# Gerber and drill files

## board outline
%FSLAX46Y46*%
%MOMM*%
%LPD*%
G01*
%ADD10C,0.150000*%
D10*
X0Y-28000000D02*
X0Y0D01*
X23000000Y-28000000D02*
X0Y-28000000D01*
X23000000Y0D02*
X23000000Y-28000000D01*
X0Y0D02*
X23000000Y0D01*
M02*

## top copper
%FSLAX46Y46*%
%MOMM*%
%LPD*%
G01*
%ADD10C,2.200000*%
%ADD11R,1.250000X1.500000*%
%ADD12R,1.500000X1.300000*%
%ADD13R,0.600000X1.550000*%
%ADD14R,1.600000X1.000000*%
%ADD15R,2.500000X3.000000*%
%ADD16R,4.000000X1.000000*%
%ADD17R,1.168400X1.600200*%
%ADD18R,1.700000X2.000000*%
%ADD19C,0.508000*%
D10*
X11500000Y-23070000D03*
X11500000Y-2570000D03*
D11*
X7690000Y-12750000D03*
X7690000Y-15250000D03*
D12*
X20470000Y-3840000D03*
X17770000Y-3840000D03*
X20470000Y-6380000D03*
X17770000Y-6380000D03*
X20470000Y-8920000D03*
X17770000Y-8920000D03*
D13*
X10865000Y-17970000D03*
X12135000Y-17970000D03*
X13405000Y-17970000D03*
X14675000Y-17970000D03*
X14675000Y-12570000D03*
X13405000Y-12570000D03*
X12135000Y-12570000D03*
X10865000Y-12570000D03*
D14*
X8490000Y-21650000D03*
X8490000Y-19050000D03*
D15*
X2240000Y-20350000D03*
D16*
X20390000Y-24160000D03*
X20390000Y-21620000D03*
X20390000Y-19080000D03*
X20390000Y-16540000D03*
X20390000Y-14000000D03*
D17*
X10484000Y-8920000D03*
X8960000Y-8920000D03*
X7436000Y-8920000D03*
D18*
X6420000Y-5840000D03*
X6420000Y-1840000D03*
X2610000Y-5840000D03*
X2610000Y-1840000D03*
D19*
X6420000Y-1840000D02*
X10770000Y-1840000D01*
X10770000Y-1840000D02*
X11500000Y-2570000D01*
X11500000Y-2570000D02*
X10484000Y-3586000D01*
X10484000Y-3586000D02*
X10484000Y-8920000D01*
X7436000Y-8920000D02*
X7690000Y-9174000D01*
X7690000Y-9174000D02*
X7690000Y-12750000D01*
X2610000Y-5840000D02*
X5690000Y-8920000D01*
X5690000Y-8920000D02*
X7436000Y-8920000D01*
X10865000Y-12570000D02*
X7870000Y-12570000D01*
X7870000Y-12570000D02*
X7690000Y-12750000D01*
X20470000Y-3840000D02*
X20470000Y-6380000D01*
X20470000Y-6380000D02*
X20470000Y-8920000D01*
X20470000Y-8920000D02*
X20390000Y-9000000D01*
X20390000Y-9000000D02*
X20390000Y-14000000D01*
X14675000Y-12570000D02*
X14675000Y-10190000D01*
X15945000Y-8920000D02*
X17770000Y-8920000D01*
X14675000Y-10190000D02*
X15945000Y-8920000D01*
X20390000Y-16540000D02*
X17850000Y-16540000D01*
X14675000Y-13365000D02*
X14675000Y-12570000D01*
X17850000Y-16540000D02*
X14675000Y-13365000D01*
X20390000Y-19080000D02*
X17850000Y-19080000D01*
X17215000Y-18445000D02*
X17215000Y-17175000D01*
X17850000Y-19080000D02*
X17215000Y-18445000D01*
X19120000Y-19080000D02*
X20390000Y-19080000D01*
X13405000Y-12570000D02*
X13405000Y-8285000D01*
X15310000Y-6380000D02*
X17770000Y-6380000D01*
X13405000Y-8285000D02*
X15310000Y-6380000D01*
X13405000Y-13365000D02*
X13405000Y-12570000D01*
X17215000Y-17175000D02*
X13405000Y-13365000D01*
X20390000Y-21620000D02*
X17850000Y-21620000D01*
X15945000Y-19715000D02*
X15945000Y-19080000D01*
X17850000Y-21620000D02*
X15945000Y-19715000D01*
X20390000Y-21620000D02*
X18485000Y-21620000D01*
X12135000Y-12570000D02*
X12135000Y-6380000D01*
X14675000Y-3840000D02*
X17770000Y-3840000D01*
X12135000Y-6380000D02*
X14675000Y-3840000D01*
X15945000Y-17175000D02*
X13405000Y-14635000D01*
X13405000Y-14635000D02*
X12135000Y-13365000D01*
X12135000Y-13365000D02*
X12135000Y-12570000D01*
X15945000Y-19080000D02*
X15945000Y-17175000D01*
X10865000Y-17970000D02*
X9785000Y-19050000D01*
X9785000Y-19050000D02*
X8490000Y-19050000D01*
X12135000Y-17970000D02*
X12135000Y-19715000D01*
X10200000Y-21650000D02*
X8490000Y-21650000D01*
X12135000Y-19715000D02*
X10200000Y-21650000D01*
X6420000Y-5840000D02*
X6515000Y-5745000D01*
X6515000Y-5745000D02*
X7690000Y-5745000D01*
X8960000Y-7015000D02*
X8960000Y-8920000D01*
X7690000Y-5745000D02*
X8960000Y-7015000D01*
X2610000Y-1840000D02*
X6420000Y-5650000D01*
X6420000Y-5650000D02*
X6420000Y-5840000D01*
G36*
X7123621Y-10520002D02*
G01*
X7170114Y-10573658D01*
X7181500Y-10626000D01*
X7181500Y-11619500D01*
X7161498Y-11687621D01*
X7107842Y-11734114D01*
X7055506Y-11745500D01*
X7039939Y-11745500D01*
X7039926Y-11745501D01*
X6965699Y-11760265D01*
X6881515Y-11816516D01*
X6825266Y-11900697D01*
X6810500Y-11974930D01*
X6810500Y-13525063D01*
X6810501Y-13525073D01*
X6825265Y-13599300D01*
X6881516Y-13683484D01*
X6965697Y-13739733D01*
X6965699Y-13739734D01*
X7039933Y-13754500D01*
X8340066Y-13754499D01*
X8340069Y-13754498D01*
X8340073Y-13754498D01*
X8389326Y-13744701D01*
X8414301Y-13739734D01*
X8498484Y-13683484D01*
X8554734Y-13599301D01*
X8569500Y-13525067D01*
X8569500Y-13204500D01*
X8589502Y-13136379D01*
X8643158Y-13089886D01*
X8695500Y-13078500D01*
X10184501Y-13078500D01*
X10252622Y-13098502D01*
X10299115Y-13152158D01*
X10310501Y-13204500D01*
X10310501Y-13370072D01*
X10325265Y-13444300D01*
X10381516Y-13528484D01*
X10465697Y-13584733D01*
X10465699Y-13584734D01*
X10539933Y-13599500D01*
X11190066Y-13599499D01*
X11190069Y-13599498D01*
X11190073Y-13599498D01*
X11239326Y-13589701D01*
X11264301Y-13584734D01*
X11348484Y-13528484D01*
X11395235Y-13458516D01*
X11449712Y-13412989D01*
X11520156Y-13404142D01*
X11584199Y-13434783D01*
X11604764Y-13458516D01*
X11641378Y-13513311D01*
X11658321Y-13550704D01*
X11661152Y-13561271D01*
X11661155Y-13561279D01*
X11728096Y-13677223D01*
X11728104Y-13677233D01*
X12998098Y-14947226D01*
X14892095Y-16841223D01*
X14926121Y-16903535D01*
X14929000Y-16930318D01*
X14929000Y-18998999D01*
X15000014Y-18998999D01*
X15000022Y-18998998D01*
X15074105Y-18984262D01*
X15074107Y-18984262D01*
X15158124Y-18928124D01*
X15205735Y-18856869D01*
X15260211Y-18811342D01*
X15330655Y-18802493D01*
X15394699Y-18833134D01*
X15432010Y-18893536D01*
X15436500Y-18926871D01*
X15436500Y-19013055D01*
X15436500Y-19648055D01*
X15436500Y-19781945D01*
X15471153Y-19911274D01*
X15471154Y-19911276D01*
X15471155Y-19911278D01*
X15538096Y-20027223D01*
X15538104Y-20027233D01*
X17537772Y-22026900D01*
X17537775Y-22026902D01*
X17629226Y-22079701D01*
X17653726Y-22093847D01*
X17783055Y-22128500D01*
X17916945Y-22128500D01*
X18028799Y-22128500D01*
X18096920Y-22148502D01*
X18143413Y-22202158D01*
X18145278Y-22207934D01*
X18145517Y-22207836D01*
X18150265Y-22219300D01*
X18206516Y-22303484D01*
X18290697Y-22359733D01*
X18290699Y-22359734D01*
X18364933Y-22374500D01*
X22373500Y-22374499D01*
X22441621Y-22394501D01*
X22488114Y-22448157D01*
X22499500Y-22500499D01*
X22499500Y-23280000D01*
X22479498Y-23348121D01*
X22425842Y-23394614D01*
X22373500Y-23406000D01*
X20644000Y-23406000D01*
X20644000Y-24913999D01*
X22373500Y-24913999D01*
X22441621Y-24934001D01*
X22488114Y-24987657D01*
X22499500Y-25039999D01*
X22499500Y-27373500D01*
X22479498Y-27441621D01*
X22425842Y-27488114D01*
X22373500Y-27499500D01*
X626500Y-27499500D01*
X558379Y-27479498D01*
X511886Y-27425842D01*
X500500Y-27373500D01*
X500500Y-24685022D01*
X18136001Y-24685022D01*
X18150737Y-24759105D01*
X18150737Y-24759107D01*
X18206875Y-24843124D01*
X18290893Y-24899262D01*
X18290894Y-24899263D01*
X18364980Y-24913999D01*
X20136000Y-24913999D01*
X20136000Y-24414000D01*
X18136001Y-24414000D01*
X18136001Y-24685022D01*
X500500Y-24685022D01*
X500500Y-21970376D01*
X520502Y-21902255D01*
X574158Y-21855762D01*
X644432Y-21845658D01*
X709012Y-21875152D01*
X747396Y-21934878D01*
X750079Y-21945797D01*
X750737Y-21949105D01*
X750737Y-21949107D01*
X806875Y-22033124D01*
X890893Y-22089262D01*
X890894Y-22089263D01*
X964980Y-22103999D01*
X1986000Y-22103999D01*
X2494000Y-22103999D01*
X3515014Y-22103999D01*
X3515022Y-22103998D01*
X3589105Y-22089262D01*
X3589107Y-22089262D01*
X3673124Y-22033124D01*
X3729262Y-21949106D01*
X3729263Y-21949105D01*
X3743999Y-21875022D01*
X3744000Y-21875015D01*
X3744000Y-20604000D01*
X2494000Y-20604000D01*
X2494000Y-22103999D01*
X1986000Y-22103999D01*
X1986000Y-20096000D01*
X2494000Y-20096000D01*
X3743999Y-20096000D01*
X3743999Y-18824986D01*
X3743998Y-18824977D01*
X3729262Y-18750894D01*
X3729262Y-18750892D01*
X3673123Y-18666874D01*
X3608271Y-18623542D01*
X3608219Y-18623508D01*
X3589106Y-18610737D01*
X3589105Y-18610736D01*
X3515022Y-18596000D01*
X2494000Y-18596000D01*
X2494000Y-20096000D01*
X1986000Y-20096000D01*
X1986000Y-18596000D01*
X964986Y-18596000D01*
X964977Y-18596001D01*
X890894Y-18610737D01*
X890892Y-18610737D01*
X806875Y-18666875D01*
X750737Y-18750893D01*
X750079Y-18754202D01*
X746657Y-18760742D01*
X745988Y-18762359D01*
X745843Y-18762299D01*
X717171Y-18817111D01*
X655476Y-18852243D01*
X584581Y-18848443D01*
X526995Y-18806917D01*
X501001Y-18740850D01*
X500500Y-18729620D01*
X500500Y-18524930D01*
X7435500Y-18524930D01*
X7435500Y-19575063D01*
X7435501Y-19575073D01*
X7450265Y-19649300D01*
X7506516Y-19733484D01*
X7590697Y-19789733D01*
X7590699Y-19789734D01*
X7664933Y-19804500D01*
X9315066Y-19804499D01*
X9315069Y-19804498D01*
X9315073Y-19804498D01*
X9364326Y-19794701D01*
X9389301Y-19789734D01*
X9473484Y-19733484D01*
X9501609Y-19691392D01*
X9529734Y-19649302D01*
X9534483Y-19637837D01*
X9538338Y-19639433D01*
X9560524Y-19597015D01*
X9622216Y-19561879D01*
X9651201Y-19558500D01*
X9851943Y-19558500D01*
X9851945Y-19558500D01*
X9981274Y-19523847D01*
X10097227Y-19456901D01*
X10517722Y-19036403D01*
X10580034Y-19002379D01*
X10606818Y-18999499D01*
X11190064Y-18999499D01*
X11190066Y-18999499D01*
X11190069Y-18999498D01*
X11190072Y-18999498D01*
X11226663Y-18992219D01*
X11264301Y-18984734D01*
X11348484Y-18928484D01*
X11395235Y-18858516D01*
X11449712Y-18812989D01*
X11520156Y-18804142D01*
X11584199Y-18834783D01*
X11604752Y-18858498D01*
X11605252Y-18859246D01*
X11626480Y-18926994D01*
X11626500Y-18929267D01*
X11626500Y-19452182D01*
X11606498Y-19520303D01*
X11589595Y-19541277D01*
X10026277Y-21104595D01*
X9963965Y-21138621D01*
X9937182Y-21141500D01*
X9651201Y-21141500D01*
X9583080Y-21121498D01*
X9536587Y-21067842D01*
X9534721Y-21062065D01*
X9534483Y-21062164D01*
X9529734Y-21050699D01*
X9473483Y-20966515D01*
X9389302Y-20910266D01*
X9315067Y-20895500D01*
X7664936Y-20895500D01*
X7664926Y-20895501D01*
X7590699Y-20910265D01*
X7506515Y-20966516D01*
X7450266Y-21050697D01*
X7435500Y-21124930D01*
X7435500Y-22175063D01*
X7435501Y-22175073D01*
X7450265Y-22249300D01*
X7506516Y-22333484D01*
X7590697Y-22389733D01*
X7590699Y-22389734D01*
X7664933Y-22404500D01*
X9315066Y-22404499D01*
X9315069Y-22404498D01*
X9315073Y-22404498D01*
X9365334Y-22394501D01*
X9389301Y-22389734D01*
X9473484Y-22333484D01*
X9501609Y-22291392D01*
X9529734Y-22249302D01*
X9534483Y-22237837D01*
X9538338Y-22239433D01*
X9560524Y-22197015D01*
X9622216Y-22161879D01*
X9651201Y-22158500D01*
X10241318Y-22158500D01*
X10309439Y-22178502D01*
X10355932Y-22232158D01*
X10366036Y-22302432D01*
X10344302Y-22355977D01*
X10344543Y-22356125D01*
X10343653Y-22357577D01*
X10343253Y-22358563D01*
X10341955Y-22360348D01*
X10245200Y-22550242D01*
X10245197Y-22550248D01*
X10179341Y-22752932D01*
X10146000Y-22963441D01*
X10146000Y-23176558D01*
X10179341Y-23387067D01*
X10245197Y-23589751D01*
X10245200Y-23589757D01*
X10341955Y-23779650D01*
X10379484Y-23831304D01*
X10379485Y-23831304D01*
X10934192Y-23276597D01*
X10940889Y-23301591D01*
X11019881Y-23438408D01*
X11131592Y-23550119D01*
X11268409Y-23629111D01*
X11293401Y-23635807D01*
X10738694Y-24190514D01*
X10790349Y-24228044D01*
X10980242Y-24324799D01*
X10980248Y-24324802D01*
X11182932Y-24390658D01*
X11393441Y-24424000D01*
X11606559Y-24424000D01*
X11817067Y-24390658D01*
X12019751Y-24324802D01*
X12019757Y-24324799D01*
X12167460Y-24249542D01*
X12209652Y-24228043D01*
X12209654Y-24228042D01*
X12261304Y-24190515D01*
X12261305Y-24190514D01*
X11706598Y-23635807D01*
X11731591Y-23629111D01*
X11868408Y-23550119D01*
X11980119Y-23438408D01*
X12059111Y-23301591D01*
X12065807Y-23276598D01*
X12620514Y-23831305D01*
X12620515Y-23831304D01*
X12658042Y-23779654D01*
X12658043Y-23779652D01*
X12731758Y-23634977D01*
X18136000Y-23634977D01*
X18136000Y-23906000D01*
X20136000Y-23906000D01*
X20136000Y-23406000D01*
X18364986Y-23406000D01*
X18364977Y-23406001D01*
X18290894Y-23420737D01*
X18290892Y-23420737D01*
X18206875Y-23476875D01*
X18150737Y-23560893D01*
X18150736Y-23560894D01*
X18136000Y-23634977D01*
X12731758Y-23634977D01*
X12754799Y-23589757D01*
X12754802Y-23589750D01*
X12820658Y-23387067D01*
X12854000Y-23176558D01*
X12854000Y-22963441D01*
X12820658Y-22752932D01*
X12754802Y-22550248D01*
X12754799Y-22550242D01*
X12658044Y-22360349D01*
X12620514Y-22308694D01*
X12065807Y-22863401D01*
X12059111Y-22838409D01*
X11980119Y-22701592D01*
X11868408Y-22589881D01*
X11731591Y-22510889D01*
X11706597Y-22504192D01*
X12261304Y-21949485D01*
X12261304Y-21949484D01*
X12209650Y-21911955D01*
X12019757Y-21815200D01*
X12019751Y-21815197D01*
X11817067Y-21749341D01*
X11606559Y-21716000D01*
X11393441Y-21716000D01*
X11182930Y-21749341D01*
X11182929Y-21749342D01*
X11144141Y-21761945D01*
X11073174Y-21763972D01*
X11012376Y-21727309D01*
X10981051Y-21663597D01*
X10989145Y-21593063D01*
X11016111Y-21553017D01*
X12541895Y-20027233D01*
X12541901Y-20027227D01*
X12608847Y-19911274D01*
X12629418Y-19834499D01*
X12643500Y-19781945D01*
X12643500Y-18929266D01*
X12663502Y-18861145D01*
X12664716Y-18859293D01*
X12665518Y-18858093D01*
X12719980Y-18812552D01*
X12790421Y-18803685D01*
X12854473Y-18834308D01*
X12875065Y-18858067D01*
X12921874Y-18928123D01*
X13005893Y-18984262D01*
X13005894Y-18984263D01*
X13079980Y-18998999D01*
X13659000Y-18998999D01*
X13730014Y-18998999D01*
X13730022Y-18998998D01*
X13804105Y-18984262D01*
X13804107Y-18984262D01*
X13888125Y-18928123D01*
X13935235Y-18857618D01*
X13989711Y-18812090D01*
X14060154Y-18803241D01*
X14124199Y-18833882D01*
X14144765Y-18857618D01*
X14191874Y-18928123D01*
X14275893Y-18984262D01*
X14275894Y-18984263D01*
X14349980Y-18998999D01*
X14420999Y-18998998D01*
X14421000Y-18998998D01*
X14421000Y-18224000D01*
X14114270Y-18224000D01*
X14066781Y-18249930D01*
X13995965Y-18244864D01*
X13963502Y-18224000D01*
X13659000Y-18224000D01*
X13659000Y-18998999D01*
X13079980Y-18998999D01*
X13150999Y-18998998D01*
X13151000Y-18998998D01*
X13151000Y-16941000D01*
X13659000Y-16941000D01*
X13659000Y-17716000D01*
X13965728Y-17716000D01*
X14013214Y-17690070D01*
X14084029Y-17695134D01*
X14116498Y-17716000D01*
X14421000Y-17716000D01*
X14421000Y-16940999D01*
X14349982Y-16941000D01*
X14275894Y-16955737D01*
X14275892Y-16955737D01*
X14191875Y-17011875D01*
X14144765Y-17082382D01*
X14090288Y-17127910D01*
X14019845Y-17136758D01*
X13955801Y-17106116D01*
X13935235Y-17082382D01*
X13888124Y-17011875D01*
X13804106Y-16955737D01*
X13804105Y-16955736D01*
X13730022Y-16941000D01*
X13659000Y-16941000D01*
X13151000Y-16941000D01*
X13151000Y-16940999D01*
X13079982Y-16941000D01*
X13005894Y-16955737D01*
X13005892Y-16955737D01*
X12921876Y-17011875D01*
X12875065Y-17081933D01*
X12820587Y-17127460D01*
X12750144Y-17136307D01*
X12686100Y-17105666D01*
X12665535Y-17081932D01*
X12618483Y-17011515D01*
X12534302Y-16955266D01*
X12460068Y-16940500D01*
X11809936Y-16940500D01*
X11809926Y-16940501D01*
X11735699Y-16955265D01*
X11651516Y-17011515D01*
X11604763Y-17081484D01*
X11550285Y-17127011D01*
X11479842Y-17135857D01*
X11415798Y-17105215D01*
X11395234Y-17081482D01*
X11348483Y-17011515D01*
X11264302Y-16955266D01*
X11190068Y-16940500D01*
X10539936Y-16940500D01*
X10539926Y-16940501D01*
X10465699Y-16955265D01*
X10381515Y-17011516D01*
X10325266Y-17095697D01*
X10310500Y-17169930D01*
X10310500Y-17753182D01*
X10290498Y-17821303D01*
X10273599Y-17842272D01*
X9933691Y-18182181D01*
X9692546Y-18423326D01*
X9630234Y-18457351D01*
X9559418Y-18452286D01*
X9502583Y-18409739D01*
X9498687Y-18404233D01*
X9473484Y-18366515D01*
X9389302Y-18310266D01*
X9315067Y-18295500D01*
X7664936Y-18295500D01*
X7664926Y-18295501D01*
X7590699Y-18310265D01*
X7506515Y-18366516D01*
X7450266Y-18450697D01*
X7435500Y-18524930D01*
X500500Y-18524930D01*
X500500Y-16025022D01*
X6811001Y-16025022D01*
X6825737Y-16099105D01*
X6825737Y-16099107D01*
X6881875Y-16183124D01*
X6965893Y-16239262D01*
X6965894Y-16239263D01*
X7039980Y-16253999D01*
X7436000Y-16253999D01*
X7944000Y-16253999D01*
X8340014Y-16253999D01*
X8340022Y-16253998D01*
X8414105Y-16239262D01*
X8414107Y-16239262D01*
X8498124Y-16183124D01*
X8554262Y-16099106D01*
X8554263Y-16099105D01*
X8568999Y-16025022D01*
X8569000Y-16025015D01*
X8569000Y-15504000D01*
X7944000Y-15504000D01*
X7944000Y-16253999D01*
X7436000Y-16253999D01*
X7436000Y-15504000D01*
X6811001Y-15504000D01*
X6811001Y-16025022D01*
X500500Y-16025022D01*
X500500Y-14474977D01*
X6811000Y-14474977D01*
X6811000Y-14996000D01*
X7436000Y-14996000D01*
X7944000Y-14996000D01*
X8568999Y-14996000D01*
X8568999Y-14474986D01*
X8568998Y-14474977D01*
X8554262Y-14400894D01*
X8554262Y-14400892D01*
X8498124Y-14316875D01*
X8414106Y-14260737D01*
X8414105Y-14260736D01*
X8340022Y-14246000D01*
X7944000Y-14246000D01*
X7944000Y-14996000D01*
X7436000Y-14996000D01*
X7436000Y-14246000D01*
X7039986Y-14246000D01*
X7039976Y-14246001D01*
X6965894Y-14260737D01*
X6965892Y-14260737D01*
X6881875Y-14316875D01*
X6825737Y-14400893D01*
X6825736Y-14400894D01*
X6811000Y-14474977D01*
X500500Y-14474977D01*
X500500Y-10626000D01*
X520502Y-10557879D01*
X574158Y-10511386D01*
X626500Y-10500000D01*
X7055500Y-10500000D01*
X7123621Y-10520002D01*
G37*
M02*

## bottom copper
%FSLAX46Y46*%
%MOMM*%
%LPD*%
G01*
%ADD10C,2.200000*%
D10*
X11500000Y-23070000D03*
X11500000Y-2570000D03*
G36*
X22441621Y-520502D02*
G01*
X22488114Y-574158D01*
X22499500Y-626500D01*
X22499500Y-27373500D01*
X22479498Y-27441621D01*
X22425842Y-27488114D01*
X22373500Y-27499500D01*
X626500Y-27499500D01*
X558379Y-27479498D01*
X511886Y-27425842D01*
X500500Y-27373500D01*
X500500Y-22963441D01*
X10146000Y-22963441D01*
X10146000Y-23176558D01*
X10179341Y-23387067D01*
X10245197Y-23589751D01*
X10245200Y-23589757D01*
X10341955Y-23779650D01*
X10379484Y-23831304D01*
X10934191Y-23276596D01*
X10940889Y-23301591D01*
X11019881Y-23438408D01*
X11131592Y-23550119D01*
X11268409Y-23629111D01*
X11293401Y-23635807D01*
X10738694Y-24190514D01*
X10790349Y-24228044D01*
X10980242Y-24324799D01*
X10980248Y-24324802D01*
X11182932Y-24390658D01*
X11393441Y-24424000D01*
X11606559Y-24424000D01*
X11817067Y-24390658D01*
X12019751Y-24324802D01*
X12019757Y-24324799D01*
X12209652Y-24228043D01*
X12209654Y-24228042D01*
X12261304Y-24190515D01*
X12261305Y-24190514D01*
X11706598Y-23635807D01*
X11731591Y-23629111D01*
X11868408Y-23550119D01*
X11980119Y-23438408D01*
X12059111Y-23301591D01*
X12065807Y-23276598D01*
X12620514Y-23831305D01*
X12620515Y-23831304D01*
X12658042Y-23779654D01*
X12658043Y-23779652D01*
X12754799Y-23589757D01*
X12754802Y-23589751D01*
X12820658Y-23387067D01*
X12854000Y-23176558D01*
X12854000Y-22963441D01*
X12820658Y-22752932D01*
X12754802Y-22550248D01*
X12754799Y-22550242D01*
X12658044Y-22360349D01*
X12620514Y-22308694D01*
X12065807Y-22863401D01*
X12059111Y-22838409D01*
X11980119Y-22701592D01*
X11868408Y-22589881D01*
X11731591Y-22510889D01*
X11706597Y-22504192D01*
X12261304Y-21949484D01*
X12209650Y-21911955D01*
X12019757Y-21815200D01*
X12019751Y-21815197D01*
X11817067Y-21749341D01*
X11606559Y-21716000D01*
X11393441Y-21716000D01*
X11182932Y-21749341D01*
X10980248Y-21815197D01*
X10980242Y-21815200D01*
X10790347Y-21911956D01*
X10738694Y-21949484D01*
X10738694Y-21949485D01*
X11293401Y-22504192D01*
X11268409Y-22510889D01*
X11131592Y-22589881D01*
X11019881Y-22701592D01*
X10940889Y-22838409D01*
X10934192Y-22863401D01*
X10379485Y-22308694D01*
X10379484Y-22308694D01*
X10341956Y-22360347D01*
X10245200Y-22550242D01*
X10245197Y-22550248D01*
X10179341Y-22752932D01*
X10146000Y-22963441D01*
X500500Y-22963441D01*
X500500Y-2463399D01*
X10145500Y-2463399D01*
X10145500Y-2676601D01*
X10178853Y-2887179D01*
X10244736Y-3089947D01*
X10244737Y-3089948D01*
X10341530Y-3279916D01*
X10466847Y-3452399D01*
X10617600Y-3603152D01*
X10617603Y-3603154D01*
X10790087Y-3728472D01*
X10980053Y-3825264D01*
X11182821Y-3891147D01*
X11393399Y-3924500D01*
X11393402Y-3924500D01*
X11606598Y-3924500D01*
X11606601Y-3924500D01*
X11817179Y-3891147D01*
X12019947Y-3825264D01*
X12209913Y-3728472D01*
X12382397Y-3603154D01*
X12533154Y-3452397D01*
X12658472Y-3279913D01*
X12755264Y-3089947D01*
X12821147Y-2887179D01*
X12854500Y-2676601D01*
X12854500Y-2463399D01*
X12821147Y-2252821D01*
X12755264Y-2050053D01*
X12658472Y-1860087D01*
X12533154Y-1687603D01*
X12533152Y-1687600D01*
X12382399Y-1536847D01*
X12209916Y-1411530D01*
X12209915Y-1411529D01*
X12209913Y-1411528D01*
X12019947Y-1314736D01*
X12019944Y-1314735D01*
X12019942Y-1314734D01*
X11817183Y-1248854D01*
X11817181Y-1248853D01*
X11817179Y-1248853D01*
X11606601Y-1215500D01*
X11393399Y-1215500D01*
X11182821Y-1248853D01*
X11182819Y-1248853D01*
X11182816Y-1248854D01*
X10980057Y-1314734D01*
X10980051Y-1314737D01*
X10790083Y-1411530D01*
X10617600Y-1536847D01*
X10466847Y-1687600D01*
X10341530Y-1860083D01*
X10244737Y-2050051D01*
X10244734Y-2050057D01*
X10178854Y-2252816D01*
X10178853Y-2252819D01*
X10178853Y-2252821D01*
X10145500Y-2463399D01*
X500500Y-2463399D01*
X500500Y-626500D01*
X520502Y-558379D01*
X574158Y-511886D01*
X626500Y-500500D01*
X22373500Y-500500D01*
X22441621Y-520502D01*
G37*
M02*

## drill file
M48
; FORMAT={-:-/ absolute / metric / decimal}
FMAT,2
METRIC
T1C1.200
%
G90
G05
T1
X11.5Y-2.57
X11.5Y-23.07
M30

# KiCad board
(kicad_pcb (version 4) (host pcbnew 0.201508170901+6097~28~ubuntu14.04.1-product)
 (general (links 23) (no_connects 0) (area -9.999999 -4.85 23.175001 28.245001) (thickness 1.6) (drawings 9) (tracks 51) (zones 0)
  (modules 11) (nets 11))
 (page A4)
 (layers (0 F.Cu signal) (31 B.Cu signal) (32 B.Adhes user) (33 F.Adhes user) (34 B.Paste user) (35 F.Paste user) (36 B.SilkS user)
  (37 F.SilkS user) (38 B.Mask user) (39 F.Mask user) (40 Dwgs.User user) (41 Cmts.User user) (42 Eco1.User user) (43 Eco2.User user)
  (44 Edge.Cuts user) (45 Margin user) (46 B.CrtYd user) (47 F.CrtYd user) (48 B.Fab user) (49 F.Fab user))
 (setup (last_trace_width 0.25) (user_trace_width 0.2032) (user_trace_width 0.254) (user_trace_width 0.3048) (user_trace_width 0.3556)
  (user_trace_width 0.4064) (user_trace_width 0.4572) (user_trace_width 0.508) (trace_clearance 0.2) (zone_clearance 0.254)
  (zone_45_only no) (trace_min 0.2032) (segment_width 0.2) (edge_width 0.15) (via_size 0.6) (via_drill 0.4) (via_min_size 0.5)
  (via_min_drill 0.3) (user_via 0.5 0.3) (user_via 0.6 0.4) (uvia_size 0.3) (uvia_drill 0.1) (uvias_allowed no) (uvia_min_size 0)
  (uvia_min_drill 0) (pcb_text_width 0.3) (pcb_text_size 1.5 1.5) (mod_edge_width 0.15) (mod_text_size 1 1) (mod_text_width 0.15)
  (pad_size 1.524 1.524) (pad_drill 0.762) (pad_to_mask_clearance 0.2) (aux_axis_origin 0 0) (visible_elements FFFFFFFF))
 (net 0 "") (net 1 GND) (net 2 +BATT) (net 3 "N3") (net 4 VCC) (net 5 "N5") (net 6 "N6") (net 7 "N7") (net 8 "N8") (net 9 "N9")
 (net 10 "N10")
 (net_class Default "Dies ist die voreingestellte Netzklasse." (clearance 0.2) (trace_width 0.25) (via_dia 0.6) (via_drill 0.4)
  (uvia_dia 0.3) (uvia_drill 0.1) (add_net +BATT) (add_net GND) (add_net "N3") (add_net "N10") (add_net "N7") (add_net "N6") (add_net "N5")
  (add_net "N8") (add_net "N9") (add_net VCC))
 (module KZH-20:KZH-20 (layer B.Cu) (at 11.5 2.57 90)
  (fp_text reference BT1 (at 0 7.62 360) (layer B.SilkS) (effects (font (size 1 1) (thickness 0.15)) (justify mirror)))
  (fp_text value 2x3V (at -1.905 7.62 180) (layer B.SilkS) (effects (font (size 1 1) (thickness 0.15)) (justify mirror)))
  (pad 2 thru_hole circle (at -20.5 0 90) (size 2.2 2.2) (drill 1.2) (layers *.Cu *.Mask B.SilkS) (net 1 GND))
  (pad 1 thru_hole circle (at 0 0 90) (size 2.2 2.2) (drill 1.2) (layers *.Cu *.Mask B.SilkS) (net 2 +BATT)))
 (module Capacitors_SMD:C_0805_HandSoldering (layer F.Cu) (at 7.69 14 270)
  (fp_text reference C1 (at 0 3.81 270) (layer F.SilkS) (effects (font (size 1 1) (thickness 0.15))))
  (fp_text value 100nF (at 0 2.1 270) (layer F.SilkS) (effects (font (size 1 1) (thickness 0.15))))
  (pad 1 smd rect (at -1.25 0 270) (size 1.5 1.25) (layers F.Cu F.Paste F.Mask) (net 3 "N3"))
  (pad 2 smd rect (at 1.25 0 270) (size 1.5 1.25) (layers F.Cu F.Paste F.Mask) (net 1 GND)))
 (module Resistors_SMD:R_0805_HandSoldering (layer F.Cu) (at 19.12 3.84 180)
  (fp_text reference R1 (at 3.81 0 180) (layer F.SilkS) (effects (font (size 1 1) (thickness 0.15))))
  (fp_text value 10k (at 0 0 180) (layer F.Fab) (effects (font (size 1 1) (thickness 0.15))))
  (pad 1 smd rect (at -1.35 0 180) (size 1.5 1.3) (layers F.Cu F.Paste F.Mask) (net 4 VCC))
  (pad 2 smd rect (at 1.35 0 180) (size 1.5 1.3) (layers F.Cu F.Paste F.Mask) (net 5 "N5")))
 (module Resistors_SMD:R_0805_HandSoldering (layer F.Cu) (at 19.12 6.38 180)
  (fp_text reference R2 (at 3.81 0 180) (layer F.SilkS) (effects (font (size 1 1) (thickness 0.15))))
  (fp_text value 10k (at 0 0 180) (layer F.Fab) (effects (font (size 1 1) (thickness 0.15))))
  (pad 1 smd rect (at -1.35 0 180) (size 1.5 1.3) (layers F.Cu F.Paste F.Mask) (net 4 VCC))
  (pad 2 smd rect (at 1.35 0 180) (size 1.5 1.3) (layers F.Cu F.Paste F.Mask) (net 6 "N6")))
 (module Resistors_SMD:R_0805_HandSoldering (layer F.Cu) (at 19.12 8.92 180)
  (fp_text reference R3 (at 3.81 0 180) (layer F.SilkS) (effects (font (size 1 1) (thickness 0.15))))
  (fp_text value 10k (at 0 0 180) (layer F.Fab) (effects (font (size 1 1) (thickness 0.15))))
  (pad 1 smd rect (at -1.35 0 180) (size 1.5 1.3) (layers F.Cu F.Paste F.Mask) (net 4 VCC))
  (pad 2 smd rect (at 1.35 0 180) (size 1.5 1.3) (layers F.Cu F.Paste F.Mask) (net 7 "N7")))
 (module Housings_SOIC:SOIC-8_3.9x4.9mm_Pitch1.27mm (layer F.Cu) (at 12.77 15.27 90)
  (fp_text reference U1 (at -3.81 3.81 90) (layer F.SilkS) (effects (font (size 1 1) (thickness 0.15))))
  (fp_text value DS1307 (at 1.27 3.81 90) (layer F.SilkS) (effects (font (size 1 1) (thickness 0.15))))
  (pad 1 smd rect (at -2.7 -1.905 90) (size 1.55 0.6) (layers F.Cu F.Paste F.Mask) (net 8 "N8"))
  (pad 2 smd rect (at -2.7 -0.635 90) (size 1.55 0.6) (layers F.Cu F.Paste F.Mask) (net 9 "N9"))
  (pad 3 smd rect (at -2.7 0.635 90) (size 1.55 0.6) (layers F.Cu F.Paste F.Mask) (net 1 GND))
  (pad 4 smd rect (at -2.7 1.905 90) (size 1.55 0.6) (layers F.Cu F.Paste F.Mask) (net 1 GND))
  (pad 5 smd rect (at 2.7 1.905 90) (size 1.55 0.6) (layers F.Cu F.Paste F.Mask) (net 7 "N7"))
  (pad 6 smd rect (at 2.7 0.635 90) (size 1.55 0.6) (layers F.Cu F.Paste F.Mask) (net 6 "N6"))
  (pad 7 smd rect (at 2.7 -0.635 90) (size 1.55 0.6) (layers F.Cu F.Paste F.Mask) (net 5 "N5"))
  (pad 8 smd rect (at 2.7 -1.905 90) (size 1.55 0.6) (layers F.Cu F.Paste F.Mask) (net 3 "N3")))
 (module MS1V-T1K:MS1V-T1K (layer F.Cu) (at 7.69 20.35)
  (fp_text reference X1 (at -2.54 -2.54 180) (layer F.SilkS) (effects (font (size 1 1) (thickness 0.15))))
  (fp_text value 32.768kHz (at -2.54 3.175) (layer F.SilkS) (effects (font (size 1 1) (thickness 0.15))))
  (pad 1 smd rect (at 0.8 1.3) (size 1.6 1) (layers F.Cu F.Paste F.Mask) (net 9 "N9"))
  (pad 2 smd rect (at 0.8 -1.3) (size 1.6 1) (layers F.Cu F.Paste F.Mask) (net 8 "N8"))
  (pad 3 smd rect (at -5.45 0) (size 2.5 3) (layers F.Cu F.Paste F.Mask) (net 1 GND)))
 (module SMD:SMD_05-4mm (layer F.Cu) (at 20.39 14)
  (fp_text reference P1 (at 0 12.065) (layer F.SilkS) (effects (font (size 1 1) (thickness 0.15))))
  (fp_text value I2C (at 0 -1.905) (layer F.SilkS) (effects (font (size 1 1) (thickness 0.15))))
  (pad 5 connect rect (at 0 10.16) (size 4 1) (layers F.Cu F.Mask) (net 1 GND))
  (pad 4 connect rect (at 0 7.62) (size 4 1) (layers F.Cu F.Mask) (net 5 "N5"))
  (pad 3 connect rect (at 0 5.08) (size 4 1) (layers F.Cu F.Mask) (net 6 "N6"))
  (pad 2 connect rect (at 0 2.54) (size 4 1) (layers F.Cu F.Mask) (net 7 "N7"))
  (pad 1 connect rect (at 0 0) (size 4 1) (layers F.Cu F.Mask) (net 4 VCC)))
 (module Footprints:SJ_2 (layer F.Cu) (at 8.96 8.92 180)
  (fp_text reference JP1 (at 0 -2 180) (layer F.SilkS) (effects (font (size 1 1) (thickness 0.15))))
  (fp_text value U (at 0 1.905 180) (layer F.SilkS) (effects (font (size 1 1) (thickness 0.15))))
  (pad 1 smd rect (at -1.524 0 180) (size 1.1684 1.6002) (layers F.Cu F.Paste F.Mask) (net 2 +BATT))
  (pad 2 smd rect (at 0 0 180) (size 1.1684 1.6002) (layers F.Cu F.Paste F.Mask) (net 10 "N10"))
  (pad 3 smd rect (at 1.524 0 180) (size 1.1684 1.6002) (layers F.Cu F.Paste F.Mask) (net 3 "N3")))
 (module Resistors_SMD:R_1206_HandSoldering (layer F.Cu) (at 6.42 3.84 90)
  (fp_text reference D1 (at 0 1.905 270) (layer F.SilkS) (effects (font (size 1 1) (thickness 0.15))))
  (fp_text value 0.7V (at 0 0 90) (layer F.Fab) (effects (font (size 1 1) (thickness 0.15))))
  (pad 1 smd rect (at -2 0 90) (size 2 1.7) (layers F.Cu F.Paste F.Mask) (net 10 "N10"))
  (pad 2 smd rect (at 2 0 90) (size 2 1.7) (layers F.Cu F.Paste F.Mask) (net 2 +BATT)))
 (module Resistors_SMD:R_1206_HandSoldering (layer F.Cu) (at 2.61 3.84 90)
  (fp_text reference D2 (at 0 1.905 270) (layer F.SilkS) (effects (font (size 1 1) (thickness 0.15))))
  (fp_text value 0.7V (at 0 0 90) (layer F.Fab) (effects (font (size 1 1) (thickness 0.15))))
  (pad 1 smd rect (at -2 0 90) (size 2 1.7) (layers F.Cu F.Paste F.Mask) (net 3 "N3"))
  (pad 2 smd rect (at 2 0 90) (size 2 1.7) (layers F.Cu F.Paste F.Mask) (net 10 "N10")))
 (gr_line (start 0 28) (end 0 0) (angle 90) (layer Edge.Cuts) (width 0.15))
 (gr_line (start 23 28) (end 0 28) (angle 90) (layer Edge.Cuts) (width 0.15))
 (gr_line (start 23 0) (end 23 28) (angle 90) (layer Edge.Cuts) (width 0.15))
 (gr_line (start 0 0) (end 23 0) (angle 90) (layer Edge.Cuts) (width 0.15))
 (segment (start 6.42 1.84) (end 10.77 1.84) (width 0.508) (layer F.Cu) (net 2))
 (segment (start 10.77 1.84) (end 11.5 2.57) (width 0.508) (layer F.Cu) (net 2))
 (segment (start 11.5 2.57) (end 10.484 3.586) (width 0.508) (layer F.Cu) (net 2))
 (segment (start 10.484 3.586) (end 10.484 8.92) (width 0.508) (layer F.Cu) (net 2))
 (segment (start 7.436 8.92) (end 7.69 9.174) (width 0.508) (layer F.Cu) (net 3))
 (segment (start 7.69 9.174) (end 7.69 12.75) (width 0.508) (layer F.Cu) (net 3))
 (segment (start 2.61 5.84) (end 5.69 8.92) (width 0.508) (layer F.Cu) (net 3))
 (segment (start 5.69 8.92) (end 7.436 8.92) (width 0.508) (layer F.Cu) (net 3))
 (segment (start 10.865 12.57) (end 7.87 12.57) (width 0.508) (layer F.Cu) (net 3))
 (segment (start 7.87 12.57) (end 7.69 12.75) (width 0.508) (layer F.Cu) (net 3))
 (segment (start 20.47 3.84) (end 20.47 6.38) (width 0.508) (layer F.Cu) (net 4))
 (segment (start 20.47 6.38) (end 20.47 8.92) (width 0.508) (layer F.Cu) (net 4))
 (segment (start 20.47 8.92) (end 20.39 9) (width 0.508) (layer F.Cu) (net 4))
 (segment (start 20.39 9) (end 20.39 14) (width 0.508) (layer F.Cu) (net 4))
 (segment (start 14.675 12.57) (end 14.675 10.19) (width 0.508) (layer F.Cu) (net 7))
 (segment (start 15.945 8.92) (end 17.77 8.92) (width 0.508) (layer F.Cu) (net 7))
 (segment (start 14.675 10.19) (end 15.945 8.92) (width 0.508) (layer F.Cu) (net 7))
 (segment (start 20.39 16.54) (end 17.85 16.54) (width 0.508) (layer F.Cu) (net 7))
 (segment (start 14.675 13.365) (end 14.675 12.57) (width 0.508) (layer F.Cu) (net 7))
 (segment (start 17.85 16.54) (end 14.675 13.365) (width 0.508) (layer F.Cu) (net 7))
 (segment (start 20.39 19.08) (end 17.85 19.08) (width 0.508) (layer F.Cu) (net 6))
 (segment (start 17.215 18.445) (end 17.215 17.175) (width 0.508) (layer F.Cu) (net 6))
 (segment (start 17.85 19.08) (end 17.215 18.445) (width 0.508) (layer F.Cu) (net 6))
 (segment (start 19.12 19.08) (end 20.39 19.08) (width 0.508) (layer F.Cu) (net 6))
 (segment (start 13.405 12.57) (end 13.405 8.285) (width 0.508) (layer F.Cu) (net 6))
 (segment (start 15.31 6.38) (end 17.77 6.38) (width 0.508) (layer F.Cu) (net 6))
 (segment (start 13.405 8.285) (end 15.31 6.38) (width 0.508) (layer F.Cu) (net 6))
 (segment (start 13.405 13.365) (end 13.405 12.57) (width 0.508) (layer F.Cu) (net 6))
 (segment (start 17.215 17.175) (end 13.405 13.365) (width 0.508) (layer F.Cu) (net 6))
 (segment (start 20.39 21.62) (end 17.85 21.62) (width 0.508) (layer F.Cu) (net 5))
 (segment (start 15.945 19.715) (end 15.945 19.08) (width 0.508) (layer F.Cu) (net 5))
 (segment (start 17.85 21.62) (end 15.945 19.715) (width 0.508) (layer F.Cu) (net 5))
 (segment (start 20.39 21.62) (end 18.485 21.62) (width 0.508) (layer F.Cu) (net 5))
 (segment (start 12.135 12.57) (end 12.135 6.38) (width 0.508) (layer F.Cu) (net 5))
 (segment (start 14.675 3.84) (end 17.77 3.84) (width 0.508) (layer F.Cu) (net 5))
 (segment (start 12.135 6.38) (end 14.675 3.84) (width 0.508) (layer F.Cu) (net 5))
 (segment (start 15.945 17.175) (end 13.405 14.635) (width 0.508) (layer F.Cu) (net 5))
 (segment (start 13.405 14.635) (end 12.135 13.365) (width 0.508) (layer F.Cu) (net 5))
 (segment (start 12.135 13.365) (end 12.135 12.57) (width 0.508) (layer F.Cu) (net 5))
 (segment (start 15.945 19.08) (end 15.945 17.175) (width 0.508) (layer F.Cu) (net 5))
 (segment (start 10.865 17.97) (end 9.785 19.05) (width 0.508) (layer F.Cu) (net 8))
 (segment (start 9.785 19.05) (end 8.49 19.05) (width 0.508) (layer F.Cu) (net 8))
 (segment (start 12.135 17.97) (end 12.135 19.715) (width 0.508) (layer F.Cu) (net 9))
 (segment (start 10.2 21.65) (end 8.49 21.65) (width 0.508) (layer F.Cu) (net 9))
 (segment (start 12.135 19.715) (end 10.2 21.65) (width 0.508) (layer F.Cu) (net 9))
 (segment (start 6.42 5.84) (end 6.515 5.745) (width 0.508) (layer F.Cu) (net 10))
 (segment (start 6.515 5.745) (end 7.69 5.745) (width 0.508) (layer F.Cu) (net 10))
 (segment (start 8.96 7.015) (end 8.96 8.92) (width 0.508) (layer F.Cu) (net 10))
 (segment (start 7.69 5.745) (end 8.96 7.015) (width 0.508) (layer F.Cu) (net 10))
 (segment (start 2.61 1.84) (end 6.42 5.65) (width 0.508) (layer F.Cu) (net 10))
 (segment (start 6.42 5.65) (end 6.42 5.84) (width 0.508) (layer F.Cu) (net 10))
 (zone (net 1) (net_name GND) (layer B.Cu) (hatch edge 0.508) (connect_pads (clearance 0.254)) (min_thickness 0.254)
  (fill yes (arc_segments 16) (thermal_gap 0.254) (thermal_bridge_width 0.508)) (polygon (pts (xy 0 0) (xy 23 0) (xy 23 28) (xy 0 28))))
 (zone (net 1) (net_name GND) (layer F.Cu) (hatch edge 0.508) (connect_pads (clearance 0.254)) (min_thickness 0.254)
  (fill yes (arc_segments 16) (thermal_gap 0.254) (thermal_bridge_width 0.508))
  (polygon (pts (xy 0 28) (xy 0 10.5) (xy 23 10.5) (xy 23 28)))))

